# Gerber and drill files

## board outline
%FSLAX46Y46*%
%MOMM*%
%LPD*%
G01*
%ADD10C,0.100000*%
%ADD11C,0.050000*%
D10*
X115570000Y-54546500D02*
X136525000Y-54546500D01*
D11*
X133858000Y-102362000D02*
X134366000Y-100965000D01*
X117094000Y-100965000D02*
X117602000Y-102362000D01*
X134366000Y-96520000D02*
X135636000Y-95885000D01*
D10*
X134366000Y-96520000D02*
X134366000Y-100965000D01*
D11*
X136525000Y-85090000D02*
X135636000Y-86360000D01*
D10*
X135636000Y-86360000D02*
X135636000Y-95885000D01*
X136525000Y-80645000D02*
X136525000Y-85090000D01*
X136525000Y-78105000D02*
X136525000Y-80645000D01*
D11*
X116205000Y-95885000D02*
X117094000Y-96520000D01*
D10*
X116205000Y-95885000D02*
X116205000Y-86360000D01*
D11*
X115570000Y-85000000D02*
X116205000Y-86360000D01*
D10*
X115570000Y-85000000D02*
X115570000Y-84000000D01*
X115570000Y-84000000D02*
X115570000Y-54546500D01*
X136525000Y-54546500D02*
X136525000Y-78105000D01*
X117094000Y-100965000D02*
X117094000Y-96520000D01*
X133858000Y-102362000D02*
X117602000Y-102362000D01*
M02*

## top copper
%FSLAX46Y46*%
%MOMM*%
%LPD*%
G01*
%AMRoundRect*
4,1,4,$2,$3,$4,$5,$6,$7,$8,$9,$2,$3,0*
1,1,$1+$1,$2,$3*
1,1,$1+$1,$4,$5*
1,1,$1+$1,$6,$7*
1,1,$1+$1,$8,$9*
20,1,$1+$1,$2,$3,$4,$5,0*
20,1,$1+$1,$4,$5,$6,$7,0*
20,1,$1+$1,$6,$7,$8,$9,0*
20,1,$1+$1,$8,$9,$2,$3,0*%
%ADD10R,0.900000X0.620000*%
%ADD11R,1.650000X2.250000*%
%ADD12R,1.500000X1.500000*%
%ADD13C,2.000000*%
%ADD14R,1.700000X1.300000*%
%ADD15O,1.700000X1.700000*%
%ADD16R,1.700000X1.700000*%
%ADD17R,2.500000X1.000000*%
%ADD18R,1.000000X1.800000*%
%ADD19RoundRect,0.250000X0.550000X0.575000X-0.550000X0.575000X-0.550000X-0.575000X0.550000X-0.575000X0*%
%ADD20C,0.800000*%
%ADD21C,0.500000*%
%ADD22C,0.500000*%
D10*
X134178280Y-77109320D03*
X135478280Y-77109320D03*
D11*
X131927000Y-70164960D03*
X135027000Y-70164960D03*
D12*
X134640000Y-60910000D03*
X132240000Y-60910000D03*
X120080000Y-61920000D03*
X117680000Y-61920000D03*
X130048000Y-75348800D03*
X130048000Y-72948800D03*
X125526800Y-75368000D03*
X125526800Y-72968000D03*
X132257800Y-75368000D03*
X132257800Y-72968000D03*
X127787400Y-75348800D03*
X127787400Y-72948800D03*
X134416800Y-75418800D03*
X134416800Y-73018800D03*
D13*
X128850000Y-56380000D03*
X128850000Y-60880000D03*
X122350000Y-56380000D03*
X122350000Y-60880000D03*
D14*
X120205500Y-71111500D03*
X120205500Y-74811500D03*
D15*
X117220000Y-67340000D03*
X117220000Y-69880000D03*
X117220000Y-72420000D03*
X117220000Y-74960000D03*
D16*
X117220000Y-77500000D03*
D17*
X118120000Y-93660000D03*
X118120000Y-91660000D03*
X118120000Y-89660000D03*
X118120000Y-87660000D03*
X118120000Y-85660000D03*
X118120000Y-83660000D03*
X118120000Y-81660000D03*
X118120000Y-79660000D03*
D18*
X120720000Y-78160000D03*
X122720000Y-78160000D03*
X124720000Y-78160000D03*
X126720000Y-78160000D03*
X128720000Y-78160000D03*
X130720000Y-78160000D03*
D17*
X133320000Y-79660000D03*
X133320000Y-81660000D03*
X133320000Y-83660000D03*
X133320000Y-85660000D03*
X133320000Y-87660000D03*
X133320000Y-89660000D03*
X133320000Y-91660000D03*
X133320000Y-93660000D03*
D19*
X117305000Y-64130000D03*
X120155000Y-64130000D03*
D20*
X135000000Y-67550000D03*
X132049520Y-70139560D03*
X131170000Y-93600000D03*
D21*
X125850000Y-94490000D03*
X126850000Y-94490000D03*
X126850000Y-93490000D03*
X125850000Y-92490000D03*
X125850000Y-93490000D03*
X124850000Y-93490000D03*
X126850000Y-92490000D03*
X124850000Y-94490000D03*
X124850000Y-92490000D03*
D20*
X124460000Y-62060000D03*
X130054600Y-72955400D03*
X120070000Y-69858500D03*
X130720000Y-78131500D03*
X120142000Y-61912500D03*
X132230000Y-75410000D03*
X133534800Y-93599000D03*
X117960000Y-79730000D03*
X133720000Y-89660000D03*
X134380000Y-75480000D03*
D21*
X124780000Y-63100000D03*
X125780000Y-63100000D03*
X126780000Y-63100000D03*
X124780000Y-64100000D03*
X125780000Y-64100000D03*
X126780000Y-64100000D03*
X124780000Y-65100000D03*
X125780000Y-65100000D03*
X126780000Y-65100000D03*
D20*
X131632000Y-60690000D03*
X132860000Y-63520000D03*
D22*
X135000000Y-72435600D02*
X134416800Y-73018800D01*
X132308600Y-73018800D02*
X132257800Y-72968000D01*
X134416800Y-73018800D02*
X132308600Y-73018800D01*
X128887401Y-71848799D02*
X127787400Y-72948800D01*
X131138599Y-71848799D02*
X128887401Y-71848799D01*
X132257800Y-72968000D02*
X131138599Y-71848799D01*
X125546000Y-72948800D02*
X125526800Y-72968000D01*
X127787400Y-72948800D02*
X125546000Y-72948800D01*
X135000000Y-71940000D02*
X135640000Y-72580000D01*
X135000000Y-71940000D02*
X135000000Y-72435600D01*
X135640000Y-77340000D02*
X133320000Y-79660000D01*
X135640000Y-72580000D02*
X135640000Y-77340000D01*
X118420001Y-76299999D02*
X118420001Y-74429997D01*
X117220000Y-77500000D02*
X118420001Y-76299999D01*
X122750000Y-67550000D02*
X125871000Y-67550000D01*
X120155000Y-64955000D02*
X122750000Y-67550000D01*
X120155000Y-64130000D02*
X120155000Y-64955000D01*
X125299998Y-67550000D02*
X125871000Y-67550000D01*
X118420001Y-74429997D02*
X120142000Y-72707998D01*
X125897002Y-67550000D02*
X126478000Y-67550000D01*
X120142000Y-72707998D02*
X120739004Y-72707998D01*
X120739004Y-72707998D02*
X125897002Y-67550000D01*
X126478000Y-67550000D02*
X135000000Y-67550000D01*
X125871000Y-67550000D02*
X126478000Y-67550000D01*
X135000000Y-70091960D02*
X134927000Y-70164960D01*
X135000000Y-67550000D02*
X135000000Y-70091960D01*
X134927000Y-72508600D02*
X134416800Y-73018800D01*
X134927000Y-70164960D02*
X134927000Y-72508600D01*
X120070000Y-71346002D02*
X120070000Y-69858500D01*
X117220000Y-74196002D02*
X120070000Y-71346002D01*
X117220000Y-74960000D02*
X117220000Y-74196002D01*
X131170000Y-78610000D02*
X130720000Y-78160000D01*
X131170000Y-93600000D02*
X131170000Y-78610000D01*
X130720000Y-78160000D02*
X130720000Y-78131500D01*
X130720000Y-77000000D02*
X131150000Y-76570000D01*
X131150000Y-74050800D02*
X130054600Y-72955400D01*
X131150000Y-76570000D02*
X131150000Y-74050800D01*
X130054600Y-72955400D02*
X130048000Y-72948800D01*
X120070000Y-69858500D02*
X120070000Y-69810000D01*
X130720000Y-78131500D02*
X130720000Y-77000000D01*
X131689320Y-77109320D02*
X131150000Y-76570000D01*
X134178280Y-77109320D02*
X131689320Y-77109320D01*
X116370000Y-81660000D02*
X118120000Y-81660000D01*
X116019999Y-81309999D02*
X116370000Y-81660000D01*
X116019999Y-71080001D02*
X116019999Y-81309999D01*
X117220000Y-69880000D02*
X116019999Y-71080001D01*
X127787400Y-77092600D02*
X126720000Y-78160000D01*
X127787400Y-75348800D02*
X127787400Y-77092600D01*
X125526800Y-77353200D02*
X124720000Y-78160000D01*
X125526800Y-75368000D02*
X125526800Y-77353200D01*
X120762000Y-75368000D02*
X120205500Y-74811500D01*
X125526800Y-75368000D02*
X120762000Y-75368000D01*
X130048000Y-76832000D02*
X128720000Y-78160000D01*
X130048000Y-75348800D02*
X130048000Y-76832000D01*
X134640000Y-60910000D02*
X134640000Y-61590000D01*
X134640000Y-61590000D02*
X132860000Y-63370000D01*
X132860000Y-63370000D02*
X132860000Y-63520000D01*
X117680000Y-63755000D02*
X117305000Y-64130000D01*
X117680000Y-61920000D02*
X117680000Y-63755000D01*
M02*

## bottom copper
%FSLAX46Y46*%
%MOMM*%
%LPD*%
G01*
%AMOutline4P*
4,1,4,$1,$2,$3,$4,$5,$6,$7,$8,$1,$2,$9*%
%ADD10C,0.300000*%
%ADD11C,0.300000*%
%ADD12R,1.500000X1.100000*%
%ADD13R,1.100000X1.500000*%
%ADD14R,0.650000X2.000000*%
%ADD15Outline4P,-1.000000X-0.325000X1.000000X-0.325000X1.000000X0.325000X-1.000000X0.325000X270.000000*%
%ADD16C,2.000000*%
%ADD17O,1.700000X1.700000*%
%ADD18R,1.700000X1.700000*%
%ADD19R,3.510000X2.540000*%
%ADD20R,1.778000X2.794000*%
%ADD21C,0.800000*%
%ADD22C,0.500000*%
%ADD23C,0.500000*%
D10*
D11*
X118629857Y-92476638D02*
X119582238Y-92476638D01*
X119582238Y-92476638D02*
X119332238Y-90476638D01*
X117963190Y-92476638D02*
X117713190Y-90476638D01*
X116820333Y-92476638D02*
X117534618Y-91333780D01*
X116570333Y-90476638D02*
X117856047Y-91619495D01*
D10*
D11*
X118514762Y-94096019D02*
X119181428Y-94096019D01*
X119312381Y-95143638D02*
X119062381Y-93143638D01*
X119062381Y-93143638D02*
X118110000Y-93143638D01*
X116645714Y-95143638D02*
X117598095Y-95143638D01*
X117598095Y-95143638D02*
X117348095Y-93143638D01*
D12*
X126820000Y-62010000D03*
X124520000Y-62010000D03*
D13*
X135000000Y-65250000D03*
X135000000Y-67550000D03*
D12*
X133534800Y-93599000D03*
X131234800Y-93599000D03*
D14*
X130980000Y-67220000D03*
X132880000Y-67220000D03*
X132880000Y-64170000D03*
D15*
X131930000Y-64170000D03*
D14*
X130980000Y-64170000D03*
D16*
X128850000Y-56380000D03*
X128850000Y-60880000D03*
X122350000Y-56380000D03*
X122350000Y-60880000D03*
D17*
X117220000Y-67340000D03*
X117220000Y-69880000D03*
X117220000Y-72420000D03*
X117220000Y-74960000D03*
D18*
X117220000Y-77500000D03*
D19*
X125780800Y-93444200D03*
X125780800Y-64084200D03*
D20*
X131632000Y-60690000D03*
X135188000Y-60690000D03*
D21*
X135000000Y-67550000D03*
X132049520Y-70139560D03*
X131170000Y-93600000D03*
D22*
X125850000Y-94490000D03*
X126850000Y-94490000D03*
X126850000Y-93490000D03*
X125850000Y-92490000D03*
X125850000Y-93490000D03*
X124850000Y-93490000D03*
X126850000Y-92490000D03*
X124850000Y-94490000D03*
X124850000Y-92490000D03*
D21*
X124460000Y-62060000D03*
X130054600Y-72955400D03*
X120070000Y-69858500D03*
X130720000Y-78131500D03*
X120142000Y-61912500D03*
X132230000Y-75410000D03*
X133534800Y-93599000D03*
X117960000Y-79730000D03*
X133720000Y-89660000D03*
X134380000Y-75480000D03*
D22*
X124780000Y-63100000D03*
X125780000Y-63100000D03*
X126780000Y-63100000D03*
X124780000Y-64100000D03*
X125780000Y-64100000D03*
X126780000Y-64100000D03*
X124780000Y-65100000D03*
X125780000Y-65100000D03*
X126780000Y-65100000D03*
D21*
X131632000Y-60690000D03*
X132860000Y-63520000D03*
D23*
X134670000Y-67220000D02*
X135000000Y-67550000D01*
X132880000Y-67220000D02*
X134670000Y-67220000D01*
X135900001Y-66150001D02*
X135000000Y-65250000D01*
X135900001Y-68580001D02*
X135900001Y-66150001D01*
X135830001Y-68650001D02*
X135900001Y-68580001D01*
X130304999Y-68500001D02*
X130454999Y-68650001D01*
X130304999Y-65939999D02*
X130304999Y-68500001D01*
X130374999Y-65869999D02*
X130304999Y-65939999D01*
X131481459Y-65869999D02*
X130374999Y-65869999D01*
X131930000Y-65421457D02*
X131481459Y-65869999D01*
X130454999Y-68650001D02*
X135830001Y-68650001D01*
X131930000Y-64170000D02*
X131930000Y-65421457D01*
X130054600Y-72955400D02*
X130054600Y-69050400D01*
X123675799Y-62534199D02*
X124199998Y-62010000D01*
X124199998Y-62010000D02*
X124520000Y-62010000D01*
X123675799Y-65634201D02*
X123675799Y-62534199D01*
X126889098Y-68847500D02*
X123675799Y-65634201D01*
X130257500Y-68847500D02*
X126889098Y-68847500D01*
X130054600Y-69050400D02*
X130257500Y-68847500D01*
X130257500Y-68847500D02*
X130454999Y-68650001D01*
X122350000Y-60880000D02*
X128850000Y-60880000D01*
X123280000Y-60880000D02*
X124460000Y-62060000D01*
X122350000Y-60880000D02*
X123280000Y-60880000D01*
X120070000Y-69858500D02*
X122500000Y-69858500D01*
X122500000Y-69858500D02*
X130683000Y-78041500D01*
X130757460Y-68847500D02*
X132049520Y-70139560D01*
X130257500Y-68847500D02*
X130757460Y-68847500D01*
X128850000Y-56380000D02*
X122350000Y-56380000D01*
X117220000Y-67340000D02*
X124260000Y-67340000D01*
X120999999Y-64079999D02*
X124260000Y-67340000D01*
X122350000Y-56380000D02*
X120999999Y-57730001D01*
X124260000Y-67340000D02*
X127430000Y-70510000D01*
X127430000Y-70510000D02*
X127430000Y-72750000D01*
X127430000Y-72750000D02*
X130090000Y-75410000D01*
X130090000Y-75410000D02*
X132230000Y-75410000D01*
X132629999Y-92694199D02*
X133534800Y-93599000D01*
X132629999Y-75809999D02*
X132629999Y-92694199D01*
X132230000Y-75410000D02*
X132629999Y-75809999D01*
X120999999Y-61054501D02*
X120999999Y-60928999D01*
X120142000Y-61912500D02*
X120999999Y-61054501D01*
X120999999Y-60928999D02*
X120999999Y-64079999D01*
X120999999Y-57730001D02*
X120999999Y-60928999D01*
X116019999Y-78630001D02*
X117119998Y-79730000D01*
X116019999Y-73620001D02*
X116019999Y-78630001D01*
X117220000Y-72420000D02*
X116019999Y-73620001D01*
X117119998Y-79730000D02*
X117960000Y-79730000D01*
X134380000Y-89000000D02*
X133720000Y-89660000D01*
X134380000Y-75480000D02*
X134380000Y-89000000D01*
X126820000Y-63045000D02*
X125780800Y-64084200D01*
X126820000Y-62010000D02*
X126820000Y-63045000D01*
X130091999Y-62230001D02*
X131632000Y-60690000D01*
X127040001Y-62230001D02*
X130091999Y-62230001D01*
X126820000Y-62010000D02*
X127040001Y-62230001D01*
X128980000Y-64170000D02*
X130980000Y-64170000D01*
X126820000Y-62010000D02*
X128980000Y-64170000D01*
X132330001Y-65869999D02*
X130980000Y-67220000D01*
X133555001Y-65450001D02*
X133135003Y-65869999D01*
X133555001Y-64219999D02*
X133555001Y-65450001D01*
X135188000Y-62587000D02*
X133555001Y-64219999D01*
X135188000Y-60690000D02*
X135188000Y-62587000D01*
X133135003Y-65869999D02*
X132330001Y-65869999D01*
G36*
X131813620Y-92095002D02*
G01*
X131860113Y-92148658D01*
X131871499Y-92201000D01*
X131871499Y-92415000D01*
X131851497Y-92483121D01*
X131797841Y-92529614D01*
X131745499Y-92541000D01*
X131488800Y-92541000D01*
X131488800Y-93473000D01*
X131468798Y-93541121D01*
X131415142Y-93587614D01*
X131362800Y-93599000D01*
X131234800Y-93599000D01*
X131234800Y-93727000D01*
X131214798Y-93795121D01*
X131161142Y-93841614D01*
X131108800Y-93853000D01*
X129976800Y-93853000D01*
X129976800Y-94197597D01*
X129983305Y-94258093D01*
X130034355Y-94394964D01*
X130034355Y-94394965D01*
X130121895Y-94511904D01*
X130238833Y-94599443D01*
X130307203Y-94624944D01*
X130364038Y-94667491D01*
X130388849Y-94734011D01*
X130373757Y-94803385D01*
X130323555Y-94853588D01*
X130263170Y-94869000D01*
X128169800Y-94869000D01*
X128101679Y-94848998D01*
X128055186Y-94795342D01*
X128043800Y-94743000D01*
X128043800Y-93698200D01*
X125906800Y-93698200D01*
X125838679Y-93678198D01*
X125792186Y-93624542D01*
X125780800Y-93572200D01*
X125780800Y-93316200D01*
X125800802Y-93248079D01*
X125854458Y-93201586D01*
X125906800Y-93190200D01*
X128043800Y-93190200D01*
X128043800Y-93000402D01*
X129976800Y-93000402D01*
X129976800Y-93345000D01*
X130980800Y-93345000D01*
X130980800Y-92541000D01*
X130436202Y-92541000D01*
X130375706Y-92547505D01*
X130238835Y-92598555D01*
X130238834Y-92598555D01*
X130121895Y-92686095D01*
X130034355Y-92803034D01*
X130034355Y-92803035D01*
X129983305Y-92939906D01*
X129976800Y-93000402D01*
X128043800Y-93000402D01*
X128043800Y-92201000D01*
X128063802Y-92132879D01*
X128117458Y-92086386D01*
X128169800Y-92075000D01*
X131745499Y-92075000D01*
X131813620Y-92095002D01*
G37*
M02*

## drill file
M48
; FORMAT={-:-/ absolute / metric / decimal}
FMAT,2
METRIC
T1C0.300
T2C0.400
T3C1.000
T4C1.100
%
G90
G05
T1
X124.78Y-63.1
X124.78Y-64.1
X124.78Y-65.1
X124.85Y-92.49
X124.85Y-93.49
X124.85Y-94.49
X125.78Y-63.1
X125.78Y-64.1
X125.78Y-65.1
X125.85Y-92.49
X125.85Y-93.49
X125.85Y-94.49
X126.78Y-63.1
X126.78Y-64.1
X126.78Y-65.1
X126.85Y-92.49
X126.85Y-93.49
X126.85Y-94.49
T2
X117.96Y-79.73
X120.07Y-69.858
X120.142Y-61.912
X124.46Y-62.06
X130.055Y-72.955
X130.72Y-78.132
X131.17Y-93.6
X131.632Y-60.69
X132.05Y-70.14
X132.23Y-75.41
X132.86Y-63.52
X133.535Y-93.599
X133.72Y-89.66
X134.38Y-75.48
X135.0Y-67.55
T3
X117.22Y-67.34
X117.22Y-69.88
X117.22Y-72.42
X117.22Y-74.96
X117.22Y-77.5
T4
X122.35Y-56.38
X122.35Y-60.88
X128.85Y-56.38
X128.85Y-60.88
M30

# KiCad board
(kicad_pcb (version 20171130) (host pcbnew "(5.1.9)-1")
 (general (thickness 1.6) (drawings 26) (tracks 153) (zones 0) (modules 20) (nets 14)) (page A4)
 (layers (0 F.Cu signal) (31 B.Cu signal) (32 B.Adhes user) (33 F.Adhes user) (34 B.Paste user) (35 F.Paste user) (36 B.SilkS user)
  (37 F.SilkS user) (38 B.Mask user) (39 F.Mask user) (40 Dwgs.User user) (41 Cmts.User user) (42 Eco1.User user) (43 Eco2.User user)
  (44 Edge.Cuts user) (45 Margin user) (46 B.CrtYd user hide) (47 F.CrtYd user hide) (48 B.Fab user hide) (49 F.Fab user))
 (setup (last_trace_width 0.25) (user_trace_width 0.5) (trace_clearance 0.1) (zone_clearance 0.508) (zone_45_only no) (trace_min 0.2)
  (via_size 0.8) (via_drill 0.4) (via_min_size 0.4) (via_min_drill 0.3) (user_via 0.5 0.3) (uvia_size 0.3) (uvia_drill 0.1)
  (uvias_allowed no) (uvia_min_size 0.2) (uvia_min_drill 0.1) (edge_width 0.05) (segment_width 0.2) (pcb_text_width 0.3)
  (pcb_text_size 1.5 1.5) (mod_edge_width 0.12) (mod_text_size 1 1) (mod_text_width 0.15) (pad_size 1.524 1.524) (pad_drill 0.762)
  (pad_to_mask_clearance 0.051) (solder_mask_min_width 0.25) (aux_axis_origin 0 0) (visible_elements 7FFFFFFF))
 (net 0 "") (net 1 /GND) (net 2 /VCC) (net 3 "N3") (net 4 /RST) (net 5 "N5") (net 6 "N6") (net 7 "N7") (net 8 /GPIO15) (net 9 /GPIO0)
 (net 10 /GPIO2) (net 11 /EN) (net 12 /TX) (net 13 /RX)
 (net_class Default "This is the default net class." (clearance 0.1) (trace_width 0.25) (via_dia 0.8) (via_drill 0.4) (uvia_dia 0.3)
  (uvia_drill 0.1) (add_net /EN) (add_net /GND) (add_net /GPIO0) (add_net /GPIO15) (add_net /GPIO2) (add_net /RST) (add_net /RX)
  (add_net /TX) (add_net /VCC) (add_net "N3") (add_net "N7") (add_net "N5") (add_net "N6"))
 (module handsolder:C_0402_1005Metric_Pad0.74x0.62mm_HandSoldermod (layer F.Cu) (at 134.82828 77.10932 180)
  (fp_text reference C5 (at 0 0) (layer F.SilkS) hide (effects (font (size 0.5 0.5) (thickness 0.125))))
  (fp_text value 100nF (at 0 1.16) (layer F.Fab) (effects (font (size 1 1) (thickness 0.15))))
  (pad 2 smd rect (at 0.65 0 180) (size 0.9 0.62) (layers F.Cu F.Paste F.Mask) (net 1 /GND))
  (pad 1 smd rect (at -0.65 0 180) (size 0.9 0.62) (layers F.Cu F.Paste F.Mask) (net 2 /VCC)))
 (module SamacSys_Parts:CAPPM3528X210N (layer F.Cu) (at 133.477 70.16496 180)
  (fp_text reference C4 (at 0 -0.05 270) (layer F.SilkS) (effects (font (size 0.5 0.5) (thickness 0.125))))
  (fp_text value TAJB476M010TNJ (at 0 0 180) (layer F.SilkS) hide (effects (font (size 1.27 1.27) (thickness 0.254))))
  (pad 2 smd rect (at 1.55 0 180) (size 1.65 2.25) (layers F.Cu F.Paste F.Mask) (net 1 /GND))
  (pad 1 smd rect (at -1.55 0 180) (size 1.65 2.25) (layers F.Cu F.Paste F.Mask) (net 2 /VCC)))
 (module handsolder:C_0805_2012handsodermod (layer B.Cu) (at 125.67 62.01)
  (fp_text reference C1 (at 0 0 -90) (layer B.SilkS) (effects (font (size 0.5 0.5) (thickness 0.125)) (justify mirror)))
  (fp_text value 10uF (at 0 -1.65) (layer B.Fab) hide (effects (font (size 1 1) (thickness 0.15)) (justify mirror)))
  (pad 2 smd rect (at 1.15 0) (size 1.5 1.1) (layers B.Cu B.Paste B.Mask) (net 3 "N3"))
  (pad 1 smd rect (at -1.15 0) (size 1.5 1.1) (layers B.Cu B.Paste B.Mask) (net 1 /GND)))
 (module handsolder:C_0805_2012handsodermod (layer B.Cu) (at 135 66.4 90)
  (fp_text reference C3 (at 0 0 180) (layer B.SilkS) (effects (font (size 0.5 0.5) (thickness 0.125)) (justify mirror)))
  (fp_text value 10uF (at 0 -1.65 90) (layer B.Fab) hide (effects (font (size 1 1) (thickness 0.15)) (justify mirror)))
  (pad 2 smd rect (at 1.15 0 90) (size 1.5 1.1) (layers B.Cu B.Paste B.Mask) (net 1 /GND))
  (pad 1 smd rect (at -1.15 0 90) (size 1.5 1.1) (layers B.Cu B.Paste B.Mask) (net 2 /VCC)))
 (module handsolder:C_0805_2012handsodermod (layer B.Cu) (at 132.3848 93.599)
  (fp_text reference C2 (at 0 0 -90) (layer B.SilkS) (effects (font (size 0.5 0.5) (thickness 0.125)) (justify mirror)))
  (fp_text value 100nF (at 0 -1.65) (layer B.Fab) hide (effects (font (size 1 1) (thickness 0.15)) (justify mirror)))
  (pad 2 smd rect (at 1.15 0) (size 1.5 1.1) (layers B.Cu B.Paste B.Mask) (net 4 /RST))
  (pad 1 smd rect (at -1.15 0) (size 1.5 1.1) (layers B.Cu B.Paste B.Mask) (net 1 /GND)))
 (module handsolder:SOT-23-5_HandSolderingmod (layer B.Cu) (at 131.93 65.72 270)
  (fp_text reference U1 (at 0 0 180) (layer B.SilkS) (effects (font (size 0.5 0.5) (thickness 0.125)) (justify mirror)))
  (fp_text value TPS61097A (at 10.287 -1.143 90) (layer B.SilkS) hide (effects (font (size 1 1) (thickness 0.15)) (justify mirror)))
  (pad 5 smd rect (at 1.5 0.95 270) (size 2 0.65) (layers B.Cu B.Paste B.Mask) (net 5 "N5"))
  (pad 4 smd rect (at 1.5 -0.95 270) (size 2 0.65) (layers B.Cu B.Paste B.Mask) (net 2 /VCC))
  (pad 3 smd rect (at -1.55 -0.95 270) (size 2 0.65) (layers B.Cu B.Paste B.Mask) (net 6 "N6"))
  (pad 2 smd trapezoid (at -1.55 0 270) (size 2 0.65) (layers B.Cu B.Paste B.Mask) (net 1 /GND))
  (pad 1 smd rect (at -1.55 0.95 270) (size 2 0.65) (layers B.Cu B.Paste B.Mask) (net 3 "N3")))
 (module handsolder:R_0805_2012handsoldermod (layer F.Cu) (at 133.44 60.91)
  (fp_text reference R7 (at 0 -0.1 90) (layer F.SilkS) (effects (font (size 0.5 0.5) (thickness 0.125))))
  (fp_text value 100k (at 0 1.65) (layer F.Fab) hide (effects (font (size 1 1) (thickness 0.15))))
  (pad 2 smd rect (at 1.2 0) (size 1.5 1.5) (layers F.Cu F.Paste F.Mask) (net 6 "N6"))
  (pad 1 smd rect (at -1.2 0) (size 1.5 1.5) (layers F.Cu F.Paste F.Mask) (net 3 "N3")))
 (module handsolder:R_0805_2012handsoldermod (layer F.Cu) (at 118.88 61.92)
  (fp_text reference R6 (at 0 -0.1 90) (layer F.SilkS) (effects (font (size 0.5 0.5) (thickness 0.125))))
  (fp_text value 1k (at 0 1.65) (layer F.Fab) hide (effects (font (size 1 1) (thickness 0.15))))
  (pad 2 smd rect (at 1.2 0) (size 1.5 1.5) (layers F.Cu F.Paste F.Mask) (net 4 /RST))
  (pad 1 smd rect (at -1.2 0) (size 1.5 1.5) (layers F.Cu F.Paste F.Mask) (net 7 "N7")))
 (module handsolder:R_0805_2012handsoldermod (layer F.Cu) (at 130.048 74.1488 270)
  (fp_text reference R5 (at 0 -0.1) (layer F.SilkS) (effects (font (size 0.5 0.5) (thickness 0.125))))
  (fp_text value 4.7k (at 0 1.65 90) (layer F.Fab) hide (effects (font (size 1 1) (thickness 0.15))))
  (pad 2 smd rect (at 1.2 0 270) (size 1.5 1.5) (layers F.Cu F.Paste F.Mask) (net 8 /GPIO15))
  (pad 1 smd rect (at -1.2 0 270) (size 1.5 1.5) (layers F.Cu F.Paste F.Mask) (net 1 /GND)))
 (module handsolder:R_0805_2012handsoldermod (layer F.Cu) (at 125.5268 74.168 270)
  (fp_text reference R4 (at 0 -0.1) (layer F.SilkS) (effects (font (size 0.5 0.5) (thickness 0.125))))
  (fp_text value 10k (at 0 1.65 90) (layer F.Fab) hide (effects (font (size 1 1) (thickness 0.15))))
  (pad 2 smd rect (at 1.2 0 270) (size 1.5 1.5) (layers F.Cu F.Paste F.Mask) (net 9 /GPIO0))
  (pad 1 smd rect (at -1.2 0 270) (size 1.5 1.5) (layers F.Cu F.Paste F.Mask) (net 2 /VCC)))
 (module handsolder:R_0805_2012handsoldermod (layer F.Cu) (at 132.2578 74.168 270)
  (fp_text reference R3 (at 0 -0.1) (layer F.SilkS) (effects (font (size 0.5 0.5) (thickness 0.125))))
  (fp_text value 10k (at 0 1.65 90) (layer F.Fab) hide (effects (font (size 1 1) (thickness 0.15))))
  (pad 2 smd rect (at 1.2 0 270) (size 1.5 1.5) (layers F.Cu F.Paste F.Mask) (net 4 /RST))
  (pad 1 smd rect (at -1.2 0 270) (size 1.5 1.5) (layers F.Cu F.Paste F.Mask) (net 2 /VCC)))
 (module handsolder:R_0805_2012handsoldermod (layer F.Cu) (at 127.7874 74.1488 270)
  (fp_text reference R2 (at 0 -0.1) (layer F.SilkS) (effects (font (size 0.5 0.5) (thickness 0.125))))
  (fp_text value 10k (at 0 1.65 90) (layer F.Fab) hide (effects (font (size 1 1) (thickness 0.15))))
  (pad 2 smd rect (at 1.2 0 270) (size 1.5 1.5) (layers F.Cu F.Paste F.Mask) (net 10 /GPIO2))
  (pad 1 smd rect (at -1.2 0 270) (size 1.5 1.5) (layers F.Cu F.Paste F.Mask) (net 2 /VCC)))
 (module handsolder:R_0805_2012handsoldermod (layer F.Cu) (at 134.4168 74.2188 270)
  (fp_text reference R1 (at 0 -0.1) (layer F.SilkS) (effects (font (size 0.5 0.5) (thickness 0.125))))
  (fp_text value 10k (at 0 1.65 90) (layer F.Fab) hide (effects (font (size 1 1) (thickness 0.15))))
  (pad 2 smd rect (at 1.2 0 270) (size 1.5 1.5) (layers F.Cu F.Paste F.Mask) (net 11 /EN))
  (pad 1 smd rect (at -1.2 0 270) (size 1.5 1.5) (layers F.Cu F.Paste F.Mask) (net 2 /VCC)))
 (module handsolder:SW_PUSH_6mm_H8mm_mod (layer F.Cu) (at 122.35 56.38)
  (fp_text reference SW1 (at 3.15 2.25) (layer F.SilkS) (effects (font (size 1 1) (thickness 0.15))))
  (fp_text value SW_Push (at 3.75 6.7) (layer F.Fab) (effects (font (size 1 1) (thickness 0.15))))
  (pad 1 thru_hole circle (at 6.5 0 90) (size 2 2) (drill 1.1) (layers *.Cu *.Mask) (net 4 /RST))
  (pad 2 thru_hole circle (at 6.5 4.5 90) (size 2 2) (drill 1.1) (layers *.Cu *.Mask) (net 1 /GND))
  (pad 1 thru_hole circle (at 0 0 90) (size 2 2) (drill 1.1) (layers *.Cu *.Mask) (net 4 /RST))
  (pad 2 thru_hole circle (at 0 4.5 90) (size 2 2) (drill 1.1) (layers *.Cu *.Mask) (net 1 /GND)))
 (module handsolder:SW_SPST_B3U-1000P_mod (layer F.Cu) (at 120.2055 72.9615 90)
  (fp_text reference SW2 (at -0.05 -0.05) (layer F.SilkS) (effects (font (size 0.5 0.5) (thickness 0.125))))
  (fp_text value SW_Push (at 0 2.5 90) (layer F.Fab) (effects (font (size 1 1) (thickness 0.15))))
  (pad 2 smd rect (at 1.85 0 90) (size 1.3 1.7) (layers F.Cu F.Paste F.Mask) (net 1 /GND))
  (pad 1 smd rect (at -1.85 0 90) (size 1.3 1.7) (layers F.Cu F.Paste F.Mask) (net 9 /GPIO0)))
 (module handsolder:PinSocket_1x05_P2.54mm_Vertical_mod (layer F.Cu) (at 117.22 77.5 180)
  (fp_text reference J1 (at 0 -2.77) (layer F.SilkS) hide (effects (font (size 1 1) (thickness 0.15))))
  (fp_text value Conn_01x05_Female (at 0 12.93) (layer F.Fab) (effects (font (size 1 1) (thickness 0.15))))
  (pad 5 thru_hole oval (at 0 10.16 180) (size 1.7 1.7) (drill 1) (layers *.Cu *.Mask) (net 4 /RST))
  (pad 4 thru_hole oval (at 0 7.62 180) (size 1.7 1.7) (drill 1) (layers *.Cu *.Mask) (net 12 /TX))
  (pad 3 thru_hole oval (at 0 5.08 180) (size 1.7 1.7) (drill 1) (layers *.Cu *.Mask) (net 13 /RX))
  (pad 2 thru_hole oval (at 0 2.54 180) (size 1.7 1.7) (drill 1) (layers *.Cu *.Mask) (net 1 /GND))
  (pad 1 thru_hole rect (at 0 0 180) (size 1.7 1.7) (drill 1) (layers *.Cu *.Mask) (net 2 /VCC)))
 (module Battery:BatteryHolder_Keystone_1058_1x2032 (layer B.Cu) (at 125.7808 78.7642 270)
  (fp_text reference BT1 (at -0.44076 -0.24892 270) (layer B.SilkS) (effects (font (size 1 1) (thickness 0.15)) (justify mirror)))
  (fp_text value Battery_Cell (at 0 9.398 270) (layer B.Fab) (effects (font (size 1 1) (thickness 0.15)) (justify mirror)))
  (pad 2 smd rect (at 14.68 0 270) (size 2.54 3.51) (layers B.Cu B.Paste B.Mask) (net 1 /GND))
  (pad 1 smd rect (at -14.68 0 270) (size 2.54 3.51) (layers B.Cu B.Paste B.Mask) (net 3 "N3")))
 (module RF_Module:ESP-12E (layer F.Cu) (at 125.72 90.16 180)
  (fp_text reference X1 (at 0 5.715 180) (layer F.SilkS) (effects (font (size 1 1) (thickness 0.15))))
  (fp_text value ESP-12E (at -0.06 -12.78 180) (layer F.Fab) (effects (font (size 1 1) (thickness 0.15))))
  (pad 22 smd rect (at 7.6 -3.5 180) (size 2.5 1) (layers F.Cu F.Paste F.Mask))
  (pad 21 smd rect (at 7.6 -1.5 180) (size 2.5 1) (layers F.Cu F.Paste F.Mask))
  (pad 20 smd rect (at 7.6 0.5 180) (size 2.5 1) (layers F.Cu F.Paste F.Mask))
  (pad 19 smd rect (at 7.6 2.5 180) (size 2.5 1) (layers F.Cu F.Paste F.Mask))
  (pad 18 smd rect (at 7.6 4.5 180) (size 2.5 1) (layers F.Cu F.Paste F.Mask))
  (pad 17 smd rect (at 7.6 6.5 180) (size 2.5 1) (layers F.Cu F.Paste F.Mask))
  (pad 16 smd rect (at 7.6 8.5 180) (size 2.5 1) (layers F.Cu F.Paste F.Mask) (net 12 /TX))
  (pad 15 smd rect (at 7.6 10.5 180) (size 2.5 1) (layers F.Cu F.Paste F.Mask) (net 13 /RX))
  (pad 14 smd rect (at 5 12 180) (size 1 1.8) (layers F.Cu F.Paste F.Mask))
  (pad 13 smd rect (at 3 12 180) (size 1 1.8) (layers F.Cu F.Paste F.Mask))
  (pad 12 smd rect (at 1 12 180) (size 1 1.8) (layers F.Cu F.Paste F.Mask) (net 9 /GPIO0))
  (pad 11 smd rect (at -1 12 180) (size 1 1.8) (layers F.Cu F.Paste F.Mask) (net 10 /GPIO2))
  (pad 10 smd rect (at -3 12 180) (size 1 1.8) (layers F.Cu F.Paste F.Mask) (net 8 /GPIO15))
  (pad 9 smd rect (at -5 12 180) (size 1 1.8) (layers F.Cu F.Paste F.Mask) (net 1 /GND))
  (pad 8 smd rect (at -7.6 10.5 180) (size 2.5 1) (layers F.Cu F.Paste F.Mask) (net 2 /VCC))
  (pad 7 smd rect (at -7.6 8.5 180) (size 2.5 1) (layers F.Cu F.Paste F.Mask))
  (pad 6 smd rect (at -7.6 6.5 180) (size 2.5 1) (layers F.Cu F.Paste F.Mask))
  (pad 5 smd rect (at -7.6 4.5 180) (size 2.5 1) (layers F.Cu F.Paste F.Mask))
  (pad 4 smd rect (at -7.6 2.5 180) (size 2.5 1) (layers F.Cu F.Paste F.Mask))
  (pad 3 smd rect (at -7.6 0.5 180) (size 2.5 1) (layers F.Cu F.Paste F.Mask) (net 11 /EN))
  (pad 2 smd rect (at -7.6 -1.5 180) (size 2.5 1) (layers F.Cu F.Paste F.Mask))
  (pad 1 smd rect (at -7.6 -3.5 180) (size 2.5 1) (layers F.Cu F.Paste F.Mask) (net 4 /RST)))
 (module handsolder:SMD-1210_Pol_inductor (layer B.Cu) (at 133.41 60.69)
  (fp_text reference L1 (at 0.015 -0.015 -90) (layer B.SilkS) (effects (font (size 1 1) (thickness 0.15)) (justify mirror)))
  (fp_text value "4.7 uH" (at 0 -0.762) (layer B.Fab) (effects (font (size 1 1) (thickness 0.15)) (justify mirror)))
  (pad 1 smd rect (at -1.778 0) (size 1.778 2.794) (layers B.Cu B.Paste B.Mask) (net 3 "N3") (zone_connect 2))
  (pad 2 smd rect (at 1.778 0) (size 1.778 2.794) (layers B.Cu B.Paste B.Mask) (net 5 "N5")))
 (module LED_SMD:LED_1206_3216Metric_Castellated (layer F.Cu) (at 118.73 64.13 180)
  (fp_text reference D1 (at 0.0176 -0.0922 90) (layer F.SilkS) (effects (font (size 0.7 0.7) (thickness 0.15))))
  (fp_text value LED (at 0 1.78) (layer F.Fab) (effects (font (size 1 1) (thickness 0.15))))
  (pad 2 smd roundrect (at 1.425 0 180) (size 1.6 1.65) (layers F.Cu F.Paste F.Mask) (roundrect_rratio 0.15625) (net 7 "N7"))
  (pad 1 smd roundrect (at -1.425 0 180) (size 1.6 1.65) (layers F.Cu F.Paste F.Mask) (roundrect_rratio 0.15625) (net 2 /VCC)))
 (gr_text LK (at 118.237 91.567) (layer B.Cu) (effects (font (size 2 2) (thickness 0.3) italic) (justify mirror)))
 (gr_line (start 115.57 54.5465) (end 136.525 54.5465) (layer Edge.Cuts) (width 0.1))
 (gr_line (start 133.858 102.362) (end 134.366 100.965) (layer Edge.Cuts) (width 0.05))
 (gr_line (start 117.094 100.965) (end 117.602 102.362) (layer Edge.Cuts) (width 0.05))
 (gr_line (start 134.366 96.52) (end 135.636 95.885) (layer Edge.Cuts) (width 0.05))
 (gr_line (start 134.366 96.52) (end 134.366 100.965) (layer Edge.Cuts) (width 0.1))
 (gr_line (start 136.525 85.09) (end 135.636 86.36) (layer Edge.Cuts) (width 0.05))
 (gr_line (start 135.636 86.36) (end 135.636 95.885) (layer Edge.Cuts) (width 0.1))
 (gr_line (start 136.525 80.645) (end 136.525 85.09) (layer Edge.Cuts) (width 0.1))
 (gr_line (start 136.525 78.105) (end 136.525 80.645) (layer Edge.Cuts) (width 0.1))
 (gr_line (start 116.205 95.885) (end 117.094 96.52) (layer Edge.Cuts) (width 0.05))
 (gr_line (start 116.205 95.885) (end 116.205 86.36) (layer Edge.Cuts) (width 0.1))
 (gr_line (start 115.57 85) (end 116.205 86.36) (layer Edge.Cuts) (width 0.05))
 (gr_line (start 115.57 85) (end 115.57 84) (layer Edge.Cuts) (width 0.1))
 (gr_line (start 115.57 84) (end 115.57 54.5465) (layer Edge.Cuts) (width 0.1))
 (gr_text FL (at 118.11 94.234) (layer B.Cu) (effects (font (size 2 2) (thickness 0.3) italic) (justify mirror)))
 (gr_line (start 136.525 54.5465) (end 136.525 78.105) (layer Edge.Cuts) (width 0.1))
 (gr_line (start 117.094 100.965) (end 117.094 96.52) (layer Edge.Cuts) (width 0.1))
 (gr_line (start 133.858 102.362) (end 117.602 102.362) (layer Edge.Cuts) (width 0.1))
 (segment (start 134.67 67.22) (end 135 67.55) (width 0.5) (layer B.Cu) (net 2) (status 30))
 (segment (start 132.88 67.22) (end 134.67 67.22) (width 0.5) (layer B.Cu) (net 2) (status 30))
 (via (at 135 67.55) (size 0.8) (drill 0.4) (layers F.Cu B.Cu) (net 2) (status 30))
 (segment (start 135 72.4356) (end 134.4168 73.0188) (width 0.5) (layer F.Cu) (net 2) (status 30))
 (segment (start 132.3086 73.0188) (end 132.2578 72.968) (width 0.5) (layer F.Cu) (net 2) (status 30))
 (segment (start 134.4168 73.0188) (end 132.3086 73.0188) (width 0.5) (layer F.Cu) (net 2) (status 30))
 (segment (start 128.887401 71.848799) (end 127.7874 72.9488) (width 0.5) (layer F.Cu) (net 2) (status 20))
 (segment (start 131.138599 71.848799) (end 128.887401 71.848799) (width 0.5) (layer F.Cu) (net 2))
 (segment (start 132.2578 72.968) (end 131.138599 71.848799) (width 0.5) (layer F.Cu) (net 2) (status 10))
 (segment (start 125.546 72.9488) (end 125.5268 72.968) (width 0.5) (layer F.Cu) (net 2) (status 30))
 (segment (start 127.7874 72.9488) (end 125.546 72.9488) (width 0.5) (layer F.Cu) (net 2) (status 30))
 (segment (start 135 71.94) (end 135.64 72.58) (width 0.5) (layer F.Cu) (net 2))
 (segment (start 135 71.94) (end 135 72.4356) (width 0.5) (layer F.Cu) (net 2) (status 20))
 (segment (start 135.64 77.34) (end 133.32 79.66) (width 0.5) (layer F.Cu) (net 2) (status 20))
 (segment (start 135.64 72.58) (end 135.64 77.34) (width 0.5) (layer F.Cu) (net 2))
 (segment (start 118.420001 76.299999) (end 118.420001 74.429997) (width 0.5) (layer F.Cu) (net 2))
 (segment (start 117.22 77.5) (end 118.420001 76.299999) (width 0.5) (layer F.Cu) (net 2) (status 10))
 (segment (start 122.75 67.55) (end 125.871 67.55) (width 0.5) (layer F.Cu) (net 2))
 (segment (start 120.155 64.955) (end 122.75 67.55) (width 0.5) (layer F.Cu) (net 2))
 (segment (start 120.155 64.13) (end 120.155 64.955) (width 0.5) (layer F.Cu) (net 2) (status 10))
 (segment (start 125.299998 67.55) (end 125.871 67.55) (width 0.5) (layer F.Cu) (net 2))
 (segment (start 118.420001 74.429997) (end 120.142 72.707998) (width 0.5) (layer F.Cu) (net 2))
 (segment (start 125.897002 67.55) (end 126.478 67.55) (width 0.5) (layer F.Cu) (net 2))
 (segment (start 120.142 72.707998) (end 120.739004 72.707998) (width 0.5) (layer F.Cu) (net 2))
 (segment (start 120.739004 72.707998) (end 125.897002 67.55) (width 0.5) (layer F.Cu) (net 2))
 (segment (start 126.478 67.55) (end 135 67.55) (width 0.5) (layer F.Cu) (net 2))
 (segment (start 125.871 67.55) (end 126.478 67.55) (width 0.5) (layer F.Cu) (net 2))
 (segment (start 135 70.09196) (end 134.927 70.16496) (width 0.5) (layer F.Cu) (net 2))
 (segment (start 135 67.55) (end 135 70.09196) (width 0.5) (layer F.Cu) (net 2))
 (segment (start 134.927 72.5086) (end 134.4168 73.0188) (width 0.5) (layer F.Cu) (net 2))
 (segment (start 134.927 70.16496) (end 134.927 72.5086) (width 0.5) (layer F.Cu) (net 2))
 (via (at 132.04952 70.13956) (size 0.8) (drill 0.4) (layers F.Cu B.Cu) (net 1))
 (via (at 131.17 93.6) (size 0.8) (drill 0.4) (layers F.Cu B.Cu) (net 1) (status 30))
 (via (at 125.85 94.49) (size 0.5) (drill 0.3) (layers F.Cu B.Cu) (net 1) (status 30))
 (via (at 126.85 94.49) (size 0.5) (drill 0.3) (layers F.Cu B.Cu) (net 1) (status 30))
 (via (at 126.85 93.49) (size 0.5) (drill 0.3) (layers F.Cu B.Cu) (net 1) (status 30))
 (via (at 125.85 92.49) (size 0.5) (drill 0.3) (layers F.Cu B.Cu) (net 1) (status 30))
 (via (at 125.85 93.49) (size 0.5) (drill 0.3) (layers F.Cu B.Cu) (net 1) (status 30))
 (via (at 124.85 93.49) (size 0.5) (drill 0.3) (layers F.Cu B.Cu) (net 1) (status 30))
 (via (at 126.85 92.49) (size 0.5) (drill 0.3) (layers F.Cu B.Cu) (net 1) (status 30))
 (via (at 124.85 94.49) (size 0.5) (drill 0.3) (layers F.Cu B.Cu) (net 1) (status 30))
 (via (at 124.85 92.49) (size 0.5) (drill 0.3) (layers F.Cu B.Cu) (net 1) (status 30))
 (segment (start 135.900001 66.150001) (end 135 65.25) (width 0.5) (layer B.Cu) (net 1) (status 20))
 (segment (start 135.900001 68.580001) (end 135.900001 66.150001) (width 0.5) (layer B.Cu) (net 1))
 (segment (start 135.830001 68.650001) (end 135.900001 68.580001) (width 0.5) (layer B.Cu) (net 1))
 (segment (start 130.304999 68.500001) (end 130.454999 68.650001) (width 0.5) (layer B.Cu) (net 1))
 (segment (start 130.304999 65.939999) (end 130.304999 68.500001) (width 0.5) (layer B.Cu) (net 1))
 (segment (start 130.374999 65.869999) (end 130.304999 65.939999) (width 0.5) (layer B.Cu) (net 1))
 (segment (start 131.481459 65.869999) (end 130.374999 65.869999) (width 0.5) (layer B.Cu) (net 1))
 (segment (start 131.93 65.421457) (end 131.481459 65.869999) (width 0.5) (layer B.Cu) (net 1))
 (segment (start 130.454999 68.650001) (end 135.830001 68.650001) (width 0.5) (layer B.Cu) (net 1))
 (segment (start 131.93 64.17) (end 131.93 65.421457) (width 0.5) (layer B.Cu) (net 1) (status 10))
 (segment (start 120.07 71.346002) (end 120.07 69.8585) (width 0.5) (layer F.Cu) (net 1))
 (segment (start 117.22 74.196002) (end 120.07 71.346002) (width 0.5) (layer F.Cu) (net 1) (status 10))
 (segment (start 117.22 74.96) (end 117.22 74.196002) (width 0.5) (layer F.Cu) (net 1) (status 30))
 (via (at 124.46 62.06) (size 0.8) (drill 0.4) (layers F.Cu B.Cu) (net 1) (status 30))
 (segment (start 131.17 78.61) (end 130.72 78.16) (width 0.5) (layer F.Cu) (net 1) (status 30))
 (segment (start 131.17 93.6) (end 131.17 78.61) (width 0.5) (layer F.Cu) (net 1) (status 20))
 (segment (start 130.72 78.16) (end 130.72 78.1315) (width 0.5) (layer F.Cu) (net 1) (status 30))
 (segment (start 130.72 77) (end 131.15 76.57) (width 0.5) (layer F.Cu) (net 1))
 (segment (start 131.15 74.0508) (end 130.0546 72.9554) (width 0.5) (layer F.Cu) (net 1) (status 20))
 (segment (start 131.15 76.57) (end 131.15 74.0508) (width 0.5) (layer F.Cu) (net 1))
 (segment (start 130.0546 72.9554) (end 130.048 72.9488) (width 0.5) (layer F.Cu) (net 1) (status 30))
 (via (at 130.0546 72.9554) (size 0.8) (drill 0.4) (layers F.Cu B.Cu) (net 1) (status 30))
 (segment (start 130.0546 72.9554) (end 130.0546 69.0504) (width 0.5) (layer B.Cu) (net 1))
 (segment (start 123.675799 62.534199) (end 124.199998 62.01) (width 0.5) (layer B.Cu) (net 1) (status 20))
 (segment (start 124.199998 62.01) (end 124.52 62.01) (width 0.5) (layer B.Cu) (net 1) (status 30))
 (segment (start 123.675799 65.634201) (end 123.675799 62.534199) (width 0.5) (layer B.Cu) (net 1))
 (segment (start 126.889098 68.8475) (end 123.675799 65.634201) (width 0.5) (layer B.Cu) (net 1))
 (segment (start 130.2575 68.8475) (end 126.889098 68.8475) (width 0.5) (layer B.Cu) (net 1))
 (segment (start 130.0546 69.0504) (end 130.2575 68.8475) (width 0.5) (layer B.Cu) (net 1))
 (segment (start 130.2575 68.8475) (end 130.454999 68.650001) (width 0.5) (layer B.Cu) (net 1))
 (segment (start 122.35 60.88) (end 128.85 60.88) (width 0.5) (layer B.Cu) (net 1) (status 30))
 (segment (start 123.28 60.88) (end 124.46 62.06) (width 0.5) (layer B.Cu) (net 1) (status 30))
 (segment (start 122.35 60.88) (end 123.28 60.88) (width 0.5) (layer B.Cu) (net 1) (status 30))
 (segment (start 120.07 69.8585) (end 120.07 69.81) (width 0.5) (layer F.Cu) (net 1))
 (via (at 120.07 69.8585) (size 0.8) (drill 0.4) (layers F.Cu B.Cu) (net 1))
 (segment (start 120.07 69.8585) (end 122.5 69.8585) (width 0.5) (layer B.Cu) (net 1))
 (segment (start 122.5 69.8585) (end 130.683 78.0415) (width 0.5) (layer B.Cu) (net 1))
 (segment (start 130.72 78.1315) (end 130.72 77) (width 0.5) (layer F.Cu) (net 1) (status 10))
 (via (at 130.72 78.1315) (size 0.8) (drill 0.4) (layers F.Cu B.Cu) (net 1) (status 30))
 (segment (start 130.75746 68.8475) (end 132.04952 70.13956) (width 0.5) (layer B.Cu) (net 1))
 (segment (start 130.2575 68.8475) (end 130.75746 68.8475) (width 0.5) (layer B.Cu) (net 1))
 (segment (start 131.68932 77.10932) (end 131.15 76.57) (width 0.5) (layer F.Cu) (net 1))
 (segment (start 134.17828 77.10932) (end 131.68932 77.10932) (width 0.5) (layer F.Cu) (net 1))
 (via (at 120.142 61.9125) (size 0.8) (drill 0.4) (layers F.Cu B.Cu) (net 4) (status 30))
 (segment (start 128.85 56.38) (end 122.35 56.38) (width 0.5) (layer B.Cu) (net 4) (status 30))
 (segment (start 117.22 67.34) (end 124.26 67.34) (width 0.5) (layer B.Cu) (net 4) (status 10))
 (segment (start 120.999999 64.079999) (end 124.26 67.34) (width 0.5) (layer B.Cu) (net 4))
 (segment (start 122.35 56.38) (end 120.999999 57.730001) (width 0.5) (layer B.Cu) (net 4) (status 10))
 (segment (start 124.26 67.34) (end 127.43 70.51) (width 0.5) (layer B.Cu) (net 4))
 (segment (start 127.43 70.51) (end 127.43 72.75) (width 0.5) (layer B.Cu) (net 4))
 (segment (start 127.43 72.75) (end 130.09 75.41) (width 0.5) (layer B.Cu) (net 4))
 (segment (start 130.09 75.41) (end 132.23 75.41) (width 0.5) (layer B.Cu) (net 4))
 (via (at 132.23 75.41) (size 0.8) (drill 0.4) (layers F.Cu B.Cu) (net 4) (status 30))
 (segment (start 132.629999 92.694199) (end 133.5348 93.599) (width 0.5) (layer B.Cu) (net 4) (status 20))
 (segment (start 132.629999 75.809999) (end 132.629999 92.694199) (width 0.5) (layer B.Cu) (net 4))
 (segment (start 132.23 75.41) (end 132.629999 75.809999) (width 0.5) (layer B.Cu) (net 4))
 (via (at 133.5348 93.599) (size 0.8) (drill 0.4) (layers F.Cu B.Cu) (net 4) (status 30))
 (segment (start 120.999999 61.054501) (end 120.999999 60.928999) (width 0.5) (layer B.Cu) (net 4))
 (segment (start 120.142 61.9125) (end 120.999999 61.054501) (width 0.5) (layer B.Cu) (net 4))
 (segment (start 120.999999 60.928999) (end 120.999999 64.079999) (width 0.5) (layer B.Cu) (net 4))
 (segment (start 120.999999 57.730001) (end 120.999999 60.928999) (width 0.5) (layer B.Cu) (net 4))
 (segment (start 116.019999 78.630001) (end 117.119998 79.73) (width 0.5) (layer B.Cu) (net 13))
 (segment (start 116.019999 73.620001) (end 116.019999 78.630001) (width 0.5) (layer B.Cu) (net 13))
 (segment (start 117.22 72.42) (end 116.019999 73.620001) (width 0.5) (layer B.Cu) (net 13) (status 10))
 (segment (start 117.119998 79.73) (end 117.96 79.73) (width 0.5) (layer B.Cu) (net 13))
 (via (at 117.96 79.73) (size 0.8) (drill 0.4) (layers F.Cu B.Cu) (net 13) (status 30))
 (segment (start 116.37 81.66) (end 118.12 81.66) (width 0.5) (layer F.Cu) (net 12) (status 20))
 (segment (start 116.019999 81.309999) (end 116.37 81.66) (width 0.5) (layer F.Cu) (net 12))
 (segment (start 116.019999 71.080001) (end 116.019999 81.309999) (width 0.5) (layer F.Cu) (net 12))
 (segment (start 117.22 69.88) (end 116.019999 71.080001) (width 0.5) (layer F.Cu) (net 12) (status 10))
 (via (at 133.72 89.66) (size 0.8) (drill 0.4) (layers F.Cu B.Cu) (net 11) (status 30))
 (via (at 134.38 75.48) (size 0.8) (drill 0.4) (layers F.Cu B.Cu) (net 11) (status 30))
 (segment (start 134.38 89) (end 133.72 89.66) (width 0.5) (layer B.Cu) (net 11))
 (segment (start 134.38 75.48) (end 134.38 89) (width 0.5) (layer B.Cu) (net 11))
 (segment (start 127.7874 77.0926) (end 126.72 78.16) (width 0.5) (layer F.Cu) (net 10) (status 20))
 (segment (start 127.7874 75.3488) (end 127.7874 77.0926) (width 0.5) (layer F.Cu) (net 10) (status 10))
 (segment (start 125.5268 77.3532) (end 124.72 78.16) (width 0.5) (layer F.Cu) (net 9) (status 20))
 (segment (start 125.5268 75.368) (end 125.5268 77.3532) (width 0.5) (layer F.Cu) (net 9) (status 10))
 (segment (start 120.762 75.368) (end 120.2055 74.8115) (width 0.5) (layer F.Cu) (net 9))
 (segment (start 125.5268 75.368) (end 120.762 75.368) (width 0.5) (layer F.Cu) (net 9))
 (via (at 124.78 63.1) (size 0.5) (drill 0.3) (layers F.Cu B.Cu) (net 3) (status 30))
 (via (at 125.78 63.1) (size 0.5) (drill 0.3) (layers F.Cu B.Cu) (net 3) (status 30))
 (via (at 126.78 63.1) (size 0.5) (drill 0.3) (layers F.Cu B.Cu) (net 3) (status 30))
 (via (at 124.78 64.1) (size 0.5) (drill 0.3) (layers F.Cu B.Cu) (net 3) (status 30))
 (via (at 125.78 64.1) (size 0.5) (drill 0.3) (layers F.Cu B.Cu) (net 3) (status 30))
 (via (at 126.78 64.1) (size 0.5) (drill 0.3) (layers F.Cu B.Cu) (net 3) (status 30))
 (via (at 124.78 65.1) (size 0.5) (drill 0.3) (layers F.Cu B.Cu) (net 3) (status 30))
 (via (at 125.78 65.1) (size 0.5) (drill 0.3) (layers F.Cu B.Cu) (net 3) (status 30))
 (via (at 126.78 65.1) (size 0.5) (drill 0.3) (layers F.Cu B.Cu) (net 3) (status 30))
 (segment (start 126.82 63.045) (end 125.7808 64.0842) (width 0.5) (layer B.Cu) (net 3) (status 30))
 (segment (start 126.82 62.01) (end 126.82 63.045) (width 0.5) (layer B.Cu) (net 3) (status 30))
 (segment (start 130.091999 62.230001) (end 131.632 60.69) (width 0.5) (layer B.Cu) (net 3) (status 20))
 (segment (start 127.040001 62.230001) (end 130.091999 62.230001) (width 0.5) (layer B.Cu) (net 3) (status 10))
 (segment (start 126.82 62.01) (end 127.040001 62.230001) (width 0.5) (layer B.Cu) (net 3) (status 30))
 (segment (start 128.98 64.17) (end 130.98 64.17) (width 0.5) (layer B.Cu) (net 3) (status 20))
 (segment (start 126.82 62.01) (end 128.98 64.17) (width 0.5) (layer B.Cu) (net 3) (status 10))
 (via (at 131.632 60.69) (size 0.8) (drill 0.4) (layers F.Cu B.Cu) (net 3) (status 30))
 (segment (start 132.330001 65.869999) (end 130.98 67.22) (width 0.5) (layer B.Cu) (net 5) (status 20))
 (segment (start 133.555001 65.450001) (end 133.135003 65.869999) (width 0.5) (layer B.Cu) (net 5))
 (segment (start 133.555001 64.219999) (end 133.555001 65.450001) (width 0.5) (layer B.Cu) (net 5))
 (segment (start 135.188 62.587) (end 133.555001 64.219999) (width 0.5) (layer B.Cu) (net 5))
 (segment (start 135.188 60.69) (end 135.188 62.587) (width 0.5) (layer B.Cu) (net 5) (status 10))
 (segment (start 133.135003 65.869999) (end 132.330001 65.869999) (width 0.5) (layer B.Cu) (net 5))
 (segment (start 130.048 76.832) (end 128.72 78.16) (width 0.5) (layer F.Cu) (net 8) (status 20))
 (segment (start 130.048 75.3488) (end 130.048 76.832) (width 0.5) (layer F.Cu) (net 8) (status 10))
 (segment (start 134.64 60.91) (end 134.64 61.59) (width 0.5) (layer F.Cu) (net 6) (status 30))
 (segment (start 134.64 61.59) (end 132.86 63.37) (width 0.5) (layer F.Cu) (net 6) (status 10))
 (segment (start 132.86 63.37) (end 132.86 63.52) (width 0.5) (layer F.Cu) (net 6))
 (via (at 132.86 63.52) (size 0.8) (drill 0.4) (layers F.Cu B.Cu) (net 6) (status 30))
 (segment (start 117.68 63.755) (end 117.305 64.13) (width 0.5) (layer F.Cu) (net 7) (status 30))
 (segment (start 117.68 61.92) (end 117.68 63.755) (width 0.5) (layer F.Cu) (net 7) (status 30))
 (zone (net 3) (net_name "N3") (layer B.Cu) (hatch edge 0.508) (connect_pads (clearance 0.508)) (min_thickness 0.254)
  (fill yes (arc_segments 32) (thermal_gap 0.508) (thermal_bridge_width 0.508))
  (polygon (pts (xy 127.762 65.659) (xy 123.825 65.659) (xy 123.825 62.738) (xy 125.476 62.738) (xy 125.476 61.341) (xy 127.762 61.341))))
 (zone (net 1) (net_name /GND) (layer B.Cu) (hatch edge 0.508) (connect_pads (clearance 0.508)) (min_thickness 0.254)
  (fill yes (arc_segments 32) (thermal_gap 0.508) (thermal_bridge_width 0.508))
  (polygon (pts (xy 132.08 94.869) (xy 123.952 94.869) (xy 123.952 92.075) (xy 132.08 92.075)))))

